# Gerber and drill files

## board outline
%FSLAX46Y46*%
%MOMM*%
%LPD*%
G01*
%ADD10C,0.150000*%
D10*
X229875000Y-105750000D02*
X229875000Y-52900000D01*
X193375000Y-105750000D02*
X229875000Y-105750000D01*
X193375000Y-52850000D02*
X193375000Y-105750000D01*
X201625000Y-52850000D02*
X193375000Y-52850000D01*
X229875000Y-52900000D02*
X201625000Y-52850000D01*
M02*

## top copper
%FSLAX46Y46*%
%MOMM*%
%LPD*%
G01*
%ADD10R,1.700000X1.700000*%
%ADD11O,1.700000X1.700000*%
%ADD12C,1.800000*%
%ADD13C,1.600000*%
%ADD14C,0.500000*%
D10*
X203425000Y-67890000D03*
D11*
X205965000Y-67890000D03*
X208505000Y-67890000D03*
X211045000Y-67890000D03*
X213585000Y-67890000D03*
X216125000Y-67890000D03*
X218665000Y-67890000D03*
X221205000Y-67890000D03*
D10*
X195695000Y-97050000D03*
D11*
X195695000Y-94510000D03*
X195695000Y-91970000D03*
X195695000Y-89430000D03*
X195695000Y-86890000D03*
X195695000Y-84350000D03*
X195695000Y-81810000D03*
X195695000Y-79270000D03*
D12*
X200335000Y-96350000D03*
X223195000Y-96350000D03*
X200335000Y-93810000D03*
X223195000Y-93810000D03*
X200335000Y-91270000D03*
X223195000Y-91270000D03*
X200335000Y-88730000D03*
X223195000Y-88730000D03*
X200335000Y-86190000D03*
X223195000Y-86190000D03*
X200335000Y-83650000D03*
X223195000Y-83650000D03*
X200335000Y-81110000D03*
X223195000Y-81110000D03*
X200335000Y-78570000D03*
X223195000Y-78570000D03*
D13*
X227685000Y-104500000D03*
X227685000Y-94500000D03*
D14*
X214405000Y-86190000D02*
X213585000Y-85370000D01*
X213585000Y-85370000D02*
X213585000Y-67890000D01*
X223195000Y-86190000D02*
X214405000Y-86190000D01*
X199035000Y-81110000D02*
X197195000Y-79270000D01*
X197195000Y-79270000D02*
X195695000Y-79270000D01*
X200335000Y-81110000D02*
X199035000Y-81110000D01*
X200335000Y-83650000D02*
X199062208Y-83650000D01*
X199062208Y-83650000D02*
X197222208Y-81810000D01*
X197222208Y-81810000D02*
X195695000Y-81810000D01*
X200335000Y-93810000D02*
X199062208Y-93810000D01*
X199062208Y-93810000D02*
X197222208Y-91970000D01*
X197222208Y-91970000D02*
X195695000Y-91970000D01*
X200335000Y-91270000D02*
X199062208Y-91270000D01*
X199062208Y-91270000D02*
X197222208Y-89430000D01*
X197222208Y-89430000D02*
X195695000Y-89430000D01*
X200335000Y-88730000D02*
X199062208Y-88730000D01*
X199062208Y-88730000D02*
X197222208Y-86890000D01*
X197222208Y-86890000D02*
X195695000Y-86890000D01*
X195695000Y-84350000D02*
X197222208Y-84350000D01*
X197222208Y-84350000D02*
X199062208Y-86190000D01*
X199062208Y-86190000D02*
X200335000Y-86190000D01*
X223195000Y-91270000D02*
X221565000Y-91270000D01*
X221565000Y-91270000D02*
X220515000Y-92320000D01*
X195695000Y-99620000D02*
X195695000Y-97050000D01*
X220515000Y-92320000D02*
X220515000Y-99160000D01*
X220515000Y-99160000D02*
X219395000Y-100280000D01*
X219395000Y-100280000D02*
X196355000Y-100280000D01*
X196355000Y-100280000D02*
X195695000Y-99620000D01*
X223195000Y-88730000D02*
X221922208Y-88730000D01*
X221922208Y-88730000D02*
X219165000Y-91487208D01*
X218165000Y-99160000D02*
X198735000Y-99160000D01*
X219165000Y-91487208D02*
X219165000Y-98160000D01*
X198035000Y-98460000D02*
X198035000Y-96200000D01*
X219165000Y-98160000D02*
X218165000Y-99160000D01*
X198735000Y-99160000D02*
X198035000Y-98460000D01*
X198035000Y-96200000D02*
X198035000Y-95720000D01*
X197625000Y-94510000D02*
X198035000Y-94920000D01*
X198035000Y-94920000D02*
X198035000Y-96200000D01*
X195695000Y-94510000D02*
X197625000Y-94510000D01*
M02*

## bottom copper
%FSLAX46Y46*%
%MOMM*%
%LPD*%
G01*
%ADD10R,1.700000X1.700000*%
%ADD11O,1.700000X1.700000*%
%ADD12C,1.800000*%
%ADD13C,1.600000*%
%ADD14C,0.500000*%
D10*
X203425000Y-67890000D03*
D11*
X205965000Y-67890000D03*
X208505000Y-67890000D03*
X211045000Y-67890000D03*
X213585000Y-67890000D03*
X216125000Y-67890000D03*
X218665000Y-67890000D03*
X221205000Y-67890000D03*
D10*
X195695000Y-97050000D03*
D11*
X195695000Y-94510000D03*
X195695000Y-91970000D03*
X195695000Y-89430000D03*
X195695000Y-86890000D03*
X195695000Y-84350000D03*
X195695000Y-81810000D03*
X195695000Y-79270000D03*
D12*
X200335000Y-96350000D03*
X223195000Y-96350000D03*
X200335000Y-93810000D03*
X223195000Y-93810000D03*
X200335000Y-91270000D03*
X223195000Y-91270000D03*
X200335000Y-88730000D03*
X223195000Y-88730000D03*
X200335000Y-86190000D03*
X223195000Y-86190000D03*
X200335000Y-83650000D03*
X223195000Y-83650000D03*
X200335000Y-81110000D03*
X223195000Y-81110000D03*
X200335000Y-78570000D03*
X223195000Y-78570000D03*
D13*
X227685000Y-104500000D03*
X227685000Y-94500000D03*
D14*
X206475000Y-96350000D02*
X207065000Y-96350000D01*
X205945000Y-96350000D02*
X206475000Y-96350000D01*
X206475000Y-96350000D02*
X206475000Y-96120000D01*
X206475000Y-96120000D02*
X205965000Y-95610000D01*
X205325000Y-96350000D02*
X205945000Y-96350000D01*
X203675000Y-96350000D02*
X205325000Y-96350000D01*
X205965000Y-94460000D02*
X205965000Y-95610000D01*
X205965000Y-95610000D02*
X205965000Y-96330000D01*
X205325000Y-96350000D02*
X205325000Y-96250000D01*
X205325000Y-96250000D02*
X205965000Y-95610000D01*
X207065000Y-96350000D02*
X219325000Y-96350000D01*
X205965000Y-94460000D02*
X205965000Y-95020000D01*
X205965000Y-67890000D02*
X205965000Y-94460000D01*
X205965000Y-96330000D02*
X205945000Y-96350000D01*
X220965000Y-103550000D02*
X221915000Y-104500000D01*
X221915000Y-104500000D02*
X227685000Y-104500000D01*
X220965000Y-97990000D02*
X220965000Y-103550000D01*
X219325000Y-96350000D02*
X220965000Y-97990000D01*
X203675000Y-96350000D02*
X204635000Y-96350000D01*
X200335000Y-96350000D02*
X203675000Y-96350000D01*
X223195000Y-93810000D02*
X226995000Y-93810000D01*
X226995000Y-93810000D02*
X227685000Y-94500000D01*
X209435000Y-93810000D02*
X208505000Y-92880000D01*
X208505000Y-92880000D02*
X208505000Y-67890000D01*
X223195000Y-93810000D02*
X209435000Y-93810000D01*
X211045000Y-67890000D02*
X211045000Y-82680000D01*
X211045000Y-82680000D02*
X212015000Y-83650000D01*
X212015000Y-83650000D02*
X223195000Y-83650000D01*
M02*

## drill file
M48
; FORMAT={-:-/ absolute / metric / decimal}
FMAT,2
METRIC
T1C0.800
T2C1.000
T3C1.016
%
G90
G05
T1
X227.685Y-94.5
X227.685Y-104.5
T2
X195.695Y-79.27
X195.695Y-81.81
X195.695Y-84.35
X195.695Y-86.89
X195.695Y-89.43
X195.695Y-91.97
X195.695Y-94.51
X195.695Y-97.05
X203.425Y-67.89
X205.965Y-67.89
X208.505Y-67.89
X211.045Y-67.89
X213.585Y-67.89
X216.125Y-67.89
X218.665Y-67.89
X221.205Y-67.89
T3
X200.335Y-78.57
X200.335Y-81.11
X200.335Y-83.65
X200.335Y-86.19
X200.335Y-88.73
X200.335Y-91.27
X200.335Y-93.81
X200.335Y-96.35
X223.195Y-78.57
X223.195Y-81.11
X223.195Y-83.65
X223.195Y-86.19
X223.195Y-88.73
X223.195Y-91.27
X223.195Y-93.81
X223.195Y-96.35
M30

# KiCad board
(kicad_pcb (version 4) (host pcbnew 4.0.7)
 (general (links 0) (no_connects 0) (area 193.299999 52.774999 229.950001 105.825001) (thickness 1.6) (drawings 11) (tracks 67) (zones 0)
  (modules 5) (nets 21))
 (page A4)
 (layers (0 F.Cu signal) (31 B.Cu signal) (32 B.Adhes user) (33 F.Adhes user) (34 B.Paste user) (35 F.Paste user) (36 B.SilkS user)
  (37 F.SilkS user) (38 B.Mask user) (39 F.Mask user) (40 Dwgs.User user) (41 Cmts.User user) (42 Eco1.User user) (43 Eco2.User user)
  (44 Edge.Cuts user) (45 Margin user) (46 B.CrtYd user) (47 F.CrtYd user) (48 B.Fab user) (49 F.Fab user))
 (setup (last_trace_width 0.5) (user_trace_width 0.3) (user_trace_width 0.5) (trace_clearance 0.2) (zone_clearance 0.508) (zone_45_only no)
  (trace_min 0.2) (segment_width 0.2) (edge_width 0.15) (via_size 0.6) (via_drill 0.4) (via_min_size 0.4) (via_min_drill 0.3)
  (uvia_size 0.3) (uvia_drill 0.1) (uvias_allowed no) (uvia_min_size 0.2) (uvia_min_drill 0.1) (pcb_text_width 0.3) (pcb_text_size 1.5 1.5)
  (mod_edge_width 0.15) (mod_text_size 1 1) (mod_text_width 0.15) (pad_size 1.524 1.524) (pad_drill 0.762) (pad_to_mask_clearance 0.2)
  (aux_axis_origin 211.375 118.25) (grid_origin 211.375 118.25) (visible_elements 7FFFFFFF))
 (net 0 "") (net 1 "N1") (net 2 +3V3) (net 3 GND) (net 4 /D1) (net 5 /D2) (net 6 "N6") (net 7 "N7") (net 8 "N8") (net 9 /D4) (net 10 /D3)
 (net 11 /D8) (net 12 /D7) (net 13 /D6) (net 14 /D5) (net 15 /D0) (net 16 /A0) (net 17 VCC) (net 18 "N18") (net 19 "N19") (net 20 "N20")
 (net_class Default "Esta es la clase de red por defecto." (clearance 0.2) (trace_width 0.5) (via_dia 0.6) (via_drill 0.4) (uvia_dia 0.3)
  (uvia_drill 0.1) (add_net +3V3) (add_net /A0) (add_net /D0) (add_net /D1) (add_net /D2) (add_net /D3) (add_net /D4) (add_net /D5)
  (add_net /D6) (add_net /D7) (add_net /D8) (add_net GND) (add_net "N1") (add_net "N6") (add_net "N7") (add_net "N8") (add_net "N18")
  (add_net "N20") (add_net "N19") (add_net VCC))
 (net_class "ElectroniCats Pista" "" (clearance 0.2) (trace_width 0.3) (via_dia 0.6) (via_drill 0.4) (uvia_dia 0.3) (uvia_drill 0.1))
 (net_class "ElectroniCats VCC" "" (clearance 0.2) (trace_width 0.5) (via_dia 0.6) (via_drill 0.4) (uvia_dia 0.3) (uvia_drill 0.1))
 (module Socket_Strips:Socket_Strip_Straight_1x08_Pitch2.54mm (layer F.Cu) (at 203.425 67.89 90)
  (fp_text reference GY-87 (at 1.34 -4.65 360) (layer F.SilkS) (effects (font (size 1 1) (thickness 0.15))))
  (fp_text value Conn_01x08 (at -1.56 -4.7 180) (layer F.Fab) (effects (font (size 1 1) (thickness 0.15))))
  (pad 1 thru_hole rect (at 0 0 90) (size 1.7 1.7) (drill 1) (layers *.Cu *.Mask) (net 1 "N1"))
  (pad 2 thru_hole oval (at 0 2.54 90) (size 1.7 1.7) (drill 1) (layers *.Cu *.Mask) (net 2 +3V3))
  (pad 3 thru_hole oval (at 0 5.08 90) (size 1.7 1.7) (drill 1) (layers *.Cu *.Mask) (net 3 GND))
  (pad 4 thru_hole oval (at 0 7.62 90) (size 1.7 1.7) (drill 1) (layers *.Cu *.Mask) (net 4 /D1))
  (pad 5 thru_hole oval (at 0 10.16 90) (size 1.7 1.7) (drill 1) (layers *.Cu *.Mask) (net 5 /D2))
  (pad 6 thru_hole oval (at 0 12.7 90) (size 1.7 1.7) (drill 1) (layers *.Cu *.Mask) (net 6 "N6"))
  (pad 7 thru_hole oval (at 0 15.24 90) (size 1.7 1.7) (drill 1) (layers *.Cu *.Mask) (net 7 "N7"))
  (pad 8 thru_hole oval (at 0 17.78 90) (size 1.7 1.7) (drill 1) (layers *.Cu *.Mask) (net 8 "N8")))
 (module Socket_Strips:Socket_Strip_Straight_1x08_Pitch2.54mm (layer F.Cu) (at 195.695 97.05 180)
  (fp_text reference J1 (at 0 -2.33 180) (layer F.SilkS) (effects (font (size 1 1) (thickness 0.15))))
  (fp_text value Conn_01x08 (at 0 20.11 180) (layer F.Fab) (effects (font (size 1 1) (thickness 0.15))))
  (pad 1 thru_hole rect (at 0 0 180) (size 1.7 1.7) (drill 1) (layers *.Cu *.Mask) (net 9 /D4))
  (pad 2 thru_hole oval (at 0 2.54 180) (size 1.7 1.7) (drill 1) (layers *.Cu *.Mask) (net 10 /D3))
  (pad 3 thru_hole oval (at 0 5.08 180) (size 1.7 1.7) (drill 1) (layers *.Cu *.Mask) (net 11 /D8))
  (pad 4 thru_hole oval (at 0 7.62 180) (size 1.7 1.7) (drill 1) (layers *.Cu *.Mask) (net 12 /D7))
  (pad 5 thru_hole oval (at 0 10.16 180) (size 1.7 1.7) (drill 1) (layers *.Cu *.Mask) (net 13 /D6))
  (pad 6 thru_hole oval (at 0 12.7 180) (size 1.7 1.7) (drill 1) (layers *.Cu *.Mask) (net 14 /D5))
  (pad 7 thru_hole oval (at 0 15.24 180) (size 1.7 1.7) (drill 1) (layers *.Cu *.Mask) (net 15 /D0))
  (pad 8 thru_hole oval (at 0 17.78 180) (size 1.7 1.7) (drill 1) (layers *.Cu *.Mask) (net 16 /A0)))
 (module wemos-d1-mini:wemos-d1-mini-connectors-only (layer F.Cu) (at 211.765 87.46 90)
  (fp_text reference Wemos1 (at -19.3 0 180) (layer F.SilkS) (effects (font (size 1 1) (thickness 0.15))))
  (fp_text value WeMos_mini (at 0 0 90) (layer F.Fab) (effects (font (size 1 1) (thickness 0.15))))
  (pad 16 thru_hole circle (at -8.89 -11.43 90) (size 1.8 1.8) (drill 1.016) (layers *.Cu *.Mask) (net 2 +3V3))
  (pad 1 thru_hole circle (at -8.89 11.43 90) (size 1.8 1.8) (drill 1.016) (layers *.Cu *.Mask) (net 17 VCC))
  (pad 15 thru_hole circle (at -6.35 -11.43 90) (size 1.8 1.8) (drill 1.016) (layers *.Cu *.Mask) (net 11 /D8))
  (pad 2 thru_hole circle (at -6.35 11.43 90) (size 1.8 1.8) (drill 1.016) (layers *.Cu *.Mask) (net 3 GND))
  (pad 14 thru_hole circle (at -3.81 -11.43 90) (size 1.8 1.8) (drill 1.016) (layers *.Cu *.Mask) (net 12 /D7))
  (pad 3 thru_hole circle (at -3.81 11.43 90) (size 1.8 1.8) (drill 1.016) (layers *.Cu *.Mask) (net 9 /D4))
  (pad 13 thru_hole circle (at -1.27 -11.43 90) (size 1.8 1.8) (drill 1.016) (layers *.Cu *.Mask) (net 13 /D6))
  (pad 4 thru_hole circle (at -1.27 11.43 90) (size 1.8 1.8) (drill 1.016) (layers *.Cu *.Mask) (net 10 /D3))
  (pad 12 thru_hole circle (at 1.27 -11.43 90) (size 1.8 1.8) (drill 1.016) (layers *.Cu *.Mask) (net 14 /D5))
  (pad 5 thru_hole circle (at 1.27 11.43 90) (size 1.8 1.8) (drill 1.016) (layers *.Cu *.Mask) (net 5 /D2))
  (pad 11 thru_hole circle (at 3.81 -11.43 90) (size 1.8 1.8) (drill 1.016) (layers *.Cu *.Mask) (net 15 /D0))
  (pad 6 thru_hole circle (at 3.81 11.43 90) (size 1.8 1.8) (drill 1.016) (layers *.Cu *.Mask) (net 4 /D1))
  (pad 10 thru_hole circle (at 6.35 -11.43 90) (size 1.8 1.8) (drill 1.016) (layers *.Cu *.Mask) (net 16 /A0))
  (pad 7 thru_hole circle (at 6.35 11.43 90) (size 1.8 1.8) (drill 1.016) (layers *.Cu *.Mask) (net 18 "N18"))
  (pad 9 thru_hole circle (at 8.89 -11.43 90) (size 1.8 1.8) (drill 1.016) (layers *.Cu *.Mask) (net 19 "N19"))
  (pad 8 thru_hole circle (at 8.89 11.43 90) (size 1.8 1.8) (drill 1.016) (layers *.Cu *.Mask) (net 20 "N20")))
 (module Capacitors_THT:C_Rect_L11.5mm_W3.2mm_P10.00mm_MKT (layer F.Cu) (at 227.685 104.5 90)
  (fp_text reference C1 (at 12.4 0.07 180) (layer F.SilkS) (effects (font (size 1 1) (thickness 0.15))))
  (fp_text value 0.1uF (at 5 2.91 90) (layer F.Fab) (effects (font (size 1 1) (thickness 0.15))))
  (pad 1 thru_hole circle (at 0 0 90) (size 1.6 1.6) (drill 0.8) (layers *.Cu *.Mask) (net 2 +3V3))
  (pad 2 thru_hole circle (at 10 0 90) (size 1.6 1.6) (drill 0.8) (layers *.Cu *.Mask) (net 3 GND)))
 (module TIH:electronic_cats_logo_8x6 (layer F.Cu) (at 197.875 59.75)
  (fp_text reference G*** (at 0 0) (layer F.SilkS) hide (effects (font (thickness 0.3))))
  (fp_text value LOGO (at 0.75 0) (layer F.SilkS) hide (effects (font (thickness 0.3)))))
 (gr_line (start 229.875 105.75) (end 229.875 52.9) (layer Edge.Cuts) (width 0.15))
 (gr_line (start 193.375 105.75) (end 229.875 105.75) (layer Edge.Cuts) (width 0.15))
 (gr_line (start 193.375 52.85) (end 193.375 105.75) (layer Edge.Cuts) (width 0.15))
 (gr_line (start 201.625 52.85) (end 193.375 52.85) (layer Edge.Cuts) (width 0.15))
 (gr_line (start 229.875 52.9) (end 201.625 52.85) (layer Edge.Cuts) (width 0.15))
 (segment (start 206.475 96.35) (end 207.065 96.35) (width 0.5) (layer B.Cu) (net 2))
 (segment (start 205.945 96.35) (end 206.475 96.35) (width 0.5) (layer B.Cu) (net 2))
 (segment (start 206.475 96.35) (end 206.475 96.12) (width 0.5) (layer B.Cu) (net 2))
 (segment (start 206.475 96.12) (end 205.965 95.61) (width 0.5) (layer B.Cu) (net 2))
 (segment (start 205.325 96.35) (end 205.945 96.35) (width 0.5) (layer B.Cu) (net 2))
 (segment (start 203.675 96.35) (end 205.325 96.35) (width 0.5) (layer B.Cu) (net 2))
 (segment (start 205.965 94.46) (end 205.965 95.61) (width 0.5) (layer B.Cu) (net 2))
 (segment (start 205.965 95.61) (end 205.965 96.33) (width 0.5) (layer B.Cu) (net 2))
 (segment (start 205.325 96.35) (end 205.325 96.25) (width 0.5) (layer B.Cu) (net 2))
 (segment (start 205.325 96.25) (end 205.965 95.61) (width 0.5) (layer B.Cu) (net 2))
 (segment (start 207.065 96.35) (end 219.325 96.35) (width 0.5) (layer B.Cu) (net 2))
 (segment (start 205.965 94.46) (end 205.965 95.02) (width 0.5) (layer B.Cu) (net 2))
 (segment (start 205.965 67.89) (end 205.965 94.46) (width 0.5) (layer B.Cu) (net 2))
 (segment (start 205.965 96.33) (end 205.945 96.35) (width 0.5) (layer B.Cu) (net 2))
 (segment (start 220.965 103.55) (end 221.915 104.5) (width 0.5) (layer B.Cu) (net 2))
 (segment (start 221.915 104.5) (end 227.685 104.5) (width 0.5) (layer B.Cu) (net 2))
 (segment (start 220.965 97.99) (end 220.965 103.55) (width 0.5) (layer B.Cu) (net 2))
 (segment (start 219.325 96.35) (end 220.965 97.99) (width 0.5) (layer B.Cu) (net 2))
 (segment (start 203.675 96.35) (end 204.635 96.35) (width 0.5) (layer B.Cu) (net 2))
 (segment (start 200.335 96.35) (end 203.675 96.35) (width 0.5) (layer B.Cu) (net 2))
 (segment (start 223.195 93.81) (end 226.995 93.81) (width 0.5) (layer B.Cu) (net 3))
 (segment (start 226.995 93.81) (end 227.685 94.5) (width 0.5) (layer B.Cu) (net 3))
 (segment (start 209.435 93.81) (end 208.505 92.88) (width 0.5) (layer B.Cu) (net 3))
 (segment (start 208.505 92.88) (end 208.505 67.89) (width 0.5) (layer B.Cu) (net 3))
 (segment (start 223.195 93.81) (end 209.435 93.81) (width 0.5) (layer B.Cu) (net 3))
 (segment (start 211.045 67.89) (end 211.045 82.68) (width 0.5) (layer B.Cu) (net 4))
 (segment (start 211.045 82.68) (end 212.015 83.65) (width 0.5) (layer B.Cu) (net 4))
 (segment (start 212.015 83.65) (end 223.195 83.65) (width 0.5) (layer B.Cu) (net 4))
 (segment (start 214.405 86.19) (end 213.585 85.37) (width 0.5) (layer F.Cu) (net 5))
 (segment (start 213.585 85.37) (end 213.585 67.89) (width 0.5) (layer F.Cu) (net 5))
 (segment (start 223.195 86.19) (end 214.405 86.19) (width 0.5) (layer F.Cu) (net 5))
 (segment (start 199.035 81.11) (end 197.195 79.27) (width 0.5) (layer F.Cu) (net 16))
 (segment (start 197.195 79.27) (end 195.695 79.27) (width 0.5) (layer F.Cu) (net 16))
 (segment (start 200.335 81.11) (end 199.035 81.11) (width 0.5) (layer F.Cu) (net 16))
 (segment (start 200.335 83.65) (end 199.062208 83.65) (width 0.5) (layer F.Cu) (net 15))
 (segment (start 199.062208 83.65) (end 197.222208 81.81) (width 0.5) (layer F.Cu) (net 15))
 (segment (start 197.222208 81.81) (end 195.695 81.81) (width 0.5) (layer F.Cu) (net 15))
 (segment (start 200.335 93.81) (end 199.062208 93.81) (width 0.5) (layer F.Cu) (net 11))
 (segment (start 199.062208 93.81) (end 197.222208 91.97) (width 0.5) (layer F.Cu) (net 11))
 (segment (start 197.222208 91.97) (end 195.695 91.97) (width 0.5) (layer F.Cu) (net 11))
 (segment (start 200.335 91.27) (end 199.062208 91.27) (width 0.5) (layer F.Cu) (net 12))
 (segment (start 199.062208 91.27) (end 197.222208 89.43) (width 0.5) (layer F.Cu) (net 12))
 (segment (start 197.222208 89.43) (end 195.695 89.43) (width 0.5) (layer F.Cu) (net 12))
 (segment (start 200.335 88.73) (end 199.062208 88.73) (width 0.5) (layer F.Cu) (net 13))
 (segment (start 199.062208 88.73) (end 197.222208 86.89) (width 0.5) (layer F.Cu) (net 13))
 (segment (start 197.222208 86.89) (end 195.695 86.89) (width 0.5) (layer F.Cu) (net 13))
 (segment (start 195.695 84.35) (end 197.222208 84.35) (width 0.5) (layer F.Cu) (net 14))
 (segment (start 197.222208 84.35) (end 199.062208 86.19) (width 0.5) (layer F.Cu) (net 14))
 (segment (start 199.062208 86.19) (end 200.335 86.19) (width 0.5) (layer F.Cu) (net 14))
 (segment (start 223.195 91.27) (end 221.565 91.27) (width 0.5) (layer F.Cu) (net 9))
 (segment (start 221.565 91.27) (end 220.515 92.32) (width 0.5) (layer F.Cu) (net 9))
 (segment (start 195.695 99.62) (end 195.695 97.05) (width 0.5) (layer F.Cu) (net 9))
 (segment (start 220.515 92.32) (end 220.515 99.16) (width 0.5) (layer F.Cu) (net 9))
 (segment (start 220.515 99.16) (end 219.395 100.28) (width 0.5) (layer F.Cu) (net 9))
 (segment (start 219.395 100.28) (end 196.355 100.28) (width 0.5) (layer F.Cu) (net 9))
 (segment (start 196.355 100.28) (end 195.695 99.62) (width 0.5) (layer F.Cu) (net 9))
 (segment (start 223.195 88.73) (end 221.922208 88.73) (width 0.5) (layer F.Cu) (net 10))
 (segment (start 221.922208 88.73) (end 219.165 91.487208) (width 0.5) (layer F.Cu) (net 10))
 (segment (start 218.165 99.16) (end 198.735 99.16) (width 0.5) (layer F.Cu) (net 10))
 (segment (start 219.165 91.487208) (end 219.165 98.16) (width 0.5) (layer F.Cu) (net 10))
 (segment (start 198.035 98.46) (end 198.035 96.2) (width 0.5) (layer F.Cu) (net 10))
 (segment (start 219.165 98.16) (end 218.165 99.16) (width 0.5) (layer F.Cu) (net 10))
 (segment (start 198.735 99.16) (end 198.035 98.46) (width 0.5) (layer F.Cu) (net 10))
 (segment (start 198.035 96.2) (end 198.035 95.72) (width 0.5) (layer F.Cu) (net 10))
 (segment (start 197.625 94.51) (end 198.035 94.92) (width 0.5) (layer F.Cu) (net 10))
 (segment (start 198.035 94.92) (end 198.035 96.2) (width 0.5) (layer F.Cu) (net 10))
 (segment (start 195.695 94.51) (end 197.625 94.51) (width 0.5) (layer F.Cu) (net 10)))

